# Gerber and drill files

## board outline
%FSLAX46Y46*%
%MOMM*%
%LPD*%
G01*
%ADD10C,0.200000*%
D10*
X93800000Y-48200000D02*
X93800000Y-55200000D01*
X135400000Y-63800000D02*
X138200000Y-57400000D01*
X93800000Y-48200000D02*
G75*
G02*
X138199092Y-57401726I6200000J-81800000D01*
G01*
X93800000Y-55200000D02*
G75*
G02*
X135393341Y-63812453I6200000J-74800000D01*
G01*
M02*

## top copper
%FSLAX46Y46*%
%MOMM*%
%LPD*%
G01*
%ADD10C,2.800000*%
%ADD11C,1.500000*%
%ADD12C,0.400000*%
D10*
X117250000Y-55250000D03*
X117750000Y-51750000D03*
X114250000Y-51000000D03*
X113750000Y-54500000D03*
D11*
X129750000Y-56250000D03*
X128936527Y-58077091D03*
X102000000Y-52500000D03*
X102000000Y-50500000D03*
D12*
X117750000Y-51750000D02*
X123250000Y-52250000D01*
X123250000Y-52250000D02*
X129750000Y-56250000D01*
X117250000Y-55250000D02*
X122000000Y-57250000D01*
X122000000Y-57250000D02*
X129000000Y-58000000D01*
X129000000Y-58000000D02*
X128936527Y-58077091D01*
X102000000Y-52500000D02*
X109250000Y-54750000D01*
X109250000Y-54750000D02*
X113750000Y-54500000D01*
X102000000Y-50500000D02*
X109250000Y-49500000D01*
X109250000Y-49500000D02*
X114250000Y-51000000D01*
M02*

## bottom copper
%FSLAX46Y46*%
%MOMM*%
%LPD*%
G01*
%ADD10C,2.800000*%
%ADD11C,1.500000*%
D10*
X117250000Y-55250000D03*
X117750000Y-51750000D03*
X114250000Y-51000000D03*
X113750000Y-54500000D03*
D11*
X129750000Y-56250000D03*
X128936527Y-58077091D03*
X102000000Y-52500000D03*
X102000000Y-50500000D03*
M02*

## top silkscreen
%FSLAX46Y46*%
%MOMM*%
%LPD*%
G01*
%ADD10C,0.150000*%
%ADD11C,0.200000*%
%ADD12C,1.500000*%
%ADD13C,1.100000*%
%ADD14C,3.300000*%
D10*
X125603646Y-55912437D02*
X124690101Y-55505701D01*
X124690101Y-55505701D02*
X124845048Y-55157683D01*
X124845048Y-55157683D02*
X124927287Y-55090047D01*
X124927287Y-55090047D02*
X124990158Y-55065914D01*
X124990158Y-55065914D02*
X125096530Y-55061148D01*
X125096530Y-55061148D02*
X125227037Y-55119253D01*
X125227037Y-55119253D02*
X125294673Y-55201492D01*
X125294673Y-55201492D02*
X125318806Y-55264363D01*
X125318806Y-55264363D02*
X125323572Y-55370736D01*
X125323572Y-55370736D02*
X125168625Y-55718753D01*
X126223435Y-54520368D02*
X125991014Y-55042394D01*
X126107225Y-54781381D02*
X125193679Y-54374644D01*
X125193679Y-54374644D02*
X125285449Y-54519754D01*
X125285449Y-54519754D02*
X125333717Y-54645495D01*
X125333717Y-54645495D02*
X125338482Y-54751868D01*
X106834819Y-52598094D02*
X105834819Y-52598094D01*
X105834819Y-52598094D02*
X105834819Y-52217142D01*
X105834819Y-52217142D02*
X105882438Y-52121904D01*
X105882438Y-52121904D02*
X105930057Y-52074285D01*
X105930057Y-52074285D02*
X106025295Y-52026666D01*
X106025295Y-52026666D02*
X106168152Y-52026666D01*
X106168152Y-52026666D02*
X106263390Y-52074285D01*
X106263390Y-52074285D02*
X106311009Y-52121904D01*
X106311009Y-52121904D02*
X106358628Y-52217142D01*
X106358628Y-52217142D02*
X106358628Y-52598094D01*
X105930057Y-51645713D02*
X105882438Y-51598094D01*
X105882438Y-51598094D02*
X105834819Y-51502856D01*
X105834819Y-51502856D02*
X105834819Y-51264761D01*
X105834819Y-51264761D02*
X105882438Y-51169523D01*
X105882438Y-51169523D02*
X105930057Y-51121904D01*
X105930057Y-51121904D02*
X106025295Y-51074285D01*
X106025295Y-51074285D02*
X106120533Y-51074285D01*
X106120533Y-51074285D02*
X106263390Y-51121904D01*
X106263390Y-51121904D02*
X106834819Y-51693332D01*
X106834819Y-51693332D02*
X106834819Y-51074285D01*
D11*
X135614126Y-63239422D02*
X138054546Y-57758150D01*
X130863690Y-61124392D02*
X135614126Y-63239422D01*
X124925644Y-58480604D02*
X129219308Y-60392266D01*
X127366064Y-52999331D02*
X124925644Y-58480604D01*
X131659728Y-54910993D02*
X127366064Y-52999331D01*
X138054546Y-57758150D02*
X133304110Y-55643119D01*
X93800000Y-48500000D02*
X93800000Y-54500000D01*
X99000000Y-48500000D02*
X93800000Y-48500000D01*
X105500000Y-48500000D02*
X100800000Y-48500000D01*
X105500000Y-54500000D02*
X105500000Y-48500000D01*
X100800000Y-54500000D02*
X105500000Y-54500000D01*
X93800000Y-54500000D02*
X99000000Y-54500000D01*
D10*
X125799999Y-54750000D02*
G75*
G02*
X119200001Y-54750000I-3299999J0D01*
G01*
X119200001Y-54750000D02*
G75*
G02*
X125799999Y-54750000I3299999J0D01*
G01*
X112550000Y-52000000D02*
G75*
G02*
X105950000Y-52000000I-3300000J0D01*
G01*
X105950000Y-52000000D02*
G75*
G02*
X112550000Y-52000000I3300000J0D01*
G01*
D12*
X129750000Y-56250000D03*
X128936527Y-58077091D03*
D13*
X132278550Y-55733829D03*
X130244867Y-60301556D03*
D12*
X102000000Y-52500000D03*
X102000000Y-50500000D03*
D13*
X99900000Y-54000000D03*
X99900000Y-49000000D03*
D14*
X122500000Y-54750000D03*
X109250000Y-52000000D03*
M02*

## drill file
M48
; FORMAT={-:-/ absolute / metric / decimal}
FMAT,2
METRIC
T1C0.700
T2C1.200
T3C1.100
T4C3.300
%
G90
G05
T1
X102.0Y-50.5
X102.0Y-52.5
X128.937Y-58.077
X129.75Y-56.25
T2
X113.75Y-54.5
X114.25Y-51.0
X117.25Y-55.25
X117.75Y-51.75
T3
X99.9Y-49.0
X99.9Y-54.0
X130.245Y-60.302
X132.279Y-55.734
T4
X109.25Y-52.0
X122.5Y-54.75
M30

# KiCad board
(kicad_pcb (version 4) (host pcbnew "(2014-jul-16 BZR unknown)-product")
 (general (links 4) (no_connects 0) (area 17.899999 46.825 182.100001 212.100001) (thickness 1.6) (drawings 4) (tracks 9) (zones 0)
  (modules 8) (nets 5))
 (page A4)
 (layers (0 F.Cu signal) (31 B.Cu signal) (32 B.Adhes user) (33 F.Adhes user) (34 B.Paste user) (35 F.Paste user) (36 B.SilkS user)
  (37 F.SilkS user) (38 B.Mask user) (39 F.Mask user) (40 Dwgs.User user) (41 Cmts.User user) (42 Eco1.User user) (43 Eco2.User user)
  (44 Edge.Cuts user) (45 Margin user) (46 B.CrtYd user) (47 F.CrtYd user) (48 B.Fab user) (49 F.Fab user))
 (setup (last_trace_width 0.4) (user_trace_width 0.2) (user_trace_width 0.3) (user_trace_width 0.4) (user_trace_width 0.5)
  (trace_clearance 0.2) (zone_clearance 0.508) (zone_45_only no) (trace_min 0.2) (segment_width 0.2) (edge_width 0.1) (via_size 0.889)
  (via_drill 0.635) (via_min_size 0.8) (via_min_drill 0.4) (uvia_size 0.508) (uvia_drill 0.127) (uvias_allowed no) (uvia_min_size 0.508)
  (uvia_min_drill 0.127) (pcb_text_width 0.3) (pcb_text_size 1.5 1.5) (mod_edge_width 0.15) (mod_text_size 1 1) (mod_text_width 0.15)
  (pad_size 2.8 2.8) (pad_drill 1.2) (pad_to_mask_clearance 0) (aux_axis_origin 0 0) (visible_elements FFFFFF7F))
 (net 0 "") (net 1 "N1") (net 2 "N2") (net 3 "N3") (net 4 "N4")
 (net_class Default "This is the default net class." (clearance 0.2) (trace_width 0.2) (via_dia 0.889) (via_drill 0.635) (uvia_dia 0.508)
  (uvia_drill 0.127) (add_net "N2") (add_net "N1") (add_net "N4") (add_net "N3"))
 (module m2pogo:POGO (layer F.Cu) (at 117.25 55.25)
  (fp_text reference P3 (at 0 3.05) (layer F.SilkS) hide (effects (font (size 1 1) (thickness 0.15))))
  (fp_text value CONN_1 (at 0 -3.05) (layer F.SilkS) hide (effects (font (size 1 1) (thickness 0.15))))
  (pad 1 thru_hole circle (at 0 0) (size 2.8 2.8) (drill 1.2) (layers *.Cu *.Mask) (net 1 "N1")))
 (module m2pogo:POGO (layer F.Cu) (at 117.75 51.75)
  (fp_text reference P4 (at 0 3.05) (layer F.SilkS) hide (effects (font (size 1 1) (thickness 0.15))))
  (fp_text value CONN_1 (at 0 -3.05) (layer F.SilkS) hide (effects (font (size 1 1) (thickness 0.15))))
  (pad 1 thru_hole circle (at 0 0) (size 2.8 2.8) (drill 1.2) (layers *.Cu *.Mask) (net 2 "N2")))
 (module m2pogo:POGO (layer F.Cu) (at 114.25 51)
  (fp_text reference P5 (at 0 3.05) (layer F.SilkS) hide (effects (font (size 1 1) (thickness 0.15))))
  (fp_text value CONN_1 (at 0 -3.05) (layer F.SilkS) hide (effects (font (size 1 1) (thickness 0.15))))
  (pad 1 thru_hole circle (at 0 0) (size 2.8 2.8) (drill 1.2) (layers *.Cu *.Mask) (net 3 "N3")))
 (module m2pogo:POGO (layer F.Cu) (at 113.75 54.5)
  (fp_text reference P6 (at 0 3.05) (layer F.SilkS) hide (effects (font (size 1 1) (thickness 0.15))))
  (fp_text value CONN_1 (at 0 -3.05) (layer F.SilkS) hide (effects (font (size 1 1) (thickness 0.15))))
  (pad 1 thru_hole circle (at 0 0) (size 2.8 2.8) (drill 1.2) (layers *.Cu *.Mask) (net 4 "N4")))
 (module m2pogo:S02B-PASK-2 (layer F.Cu) (at 129.75 56.25 246)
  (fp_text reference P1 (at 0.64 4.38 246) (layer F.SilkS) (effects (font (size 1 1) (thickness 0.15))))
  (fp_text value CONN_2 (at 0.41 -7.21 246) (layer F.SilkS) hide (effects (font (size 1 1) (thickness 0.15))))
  (fp_line (start 4 -8.2) (end -2 -8.2) (layer F.SilkS) (width 0.2))
  (fp_line (start 4 -3) (end 4 -8.2) (layer F.SilkS) (width 0.2))
  (fp_line (start 4 3.5) (end 4 -1.2) (layer F.SilkS) (width 0.2))
  (fp_line (start -2 3.5) (end 4 3.5) (layer F.SilkS) (width 0.2))
  (fp_line (start -2 -1.2) (end -2 3.5) (layer F.SilkS) (width 0.2))
  (fp_line (start -2 -8.2) (end -2 -3) (layer F.SilkS) (width 0.2))
  (pad 1 thru_hole circle (at 0 0 246) (size 1.5 1.5) (drill 0.7) (layers *.Cu *.Mask F.SilkS) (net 2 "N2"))
  (pad 2 thru_hole circle (at 2 0 246) (size 1.5 1.5) (drill 0.7) (layers *.Cu *.Mask F.SilkS) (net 1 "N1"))
  (pad "" np_thru_hole circle (at -1.5 -2.1 246) (size 1.1 1.1) (drill 1.1) (layers *.Cu *.Mask F.SilkS))
  (pad "" np_thru_hole circle (at 3.5 -2.1 246) (size 1.1 1.1) (drill 1.1) (layers *.Cu *.Mask F.SilkS)))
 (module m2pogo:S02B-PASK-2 (layer F.Cu) (at 102 52.5 90)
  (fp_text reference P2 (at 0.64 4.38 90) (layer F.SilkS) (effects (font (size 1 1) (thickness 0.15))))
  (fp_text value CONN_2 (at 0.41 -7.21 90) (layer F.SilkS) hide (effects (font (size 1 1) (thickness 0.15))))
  (fp_line (start 4 -8.2) (end -2 -8.2) (layer F.SilkS) (width 0.2))
  (fp_line (start 4 -3) (end 4 -8.2) (layer F.SilkS) (width 0.2))
  (fp_line (start 4 3.5) (end 4 -1.2) (layer F.SilkS) (width 0.2))
  (fp_line (start -2 3.5) (end 4 3.5) (layer F.SilkS) (width 0.2))
  (fp_line (start -2 -1.2) (end -2 3.5) (layer F.SilkS) (width 0.2))
  (fp_line (start -2 -8.2) (end -2 -3) (layer F.SilkS) (width 0.2))
  (pad 1 thru_hole circle (at 0 0 90) (size 1.5 1.5) (drill 0.7) (layers *.Cu *.Mask F.SilkS) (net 4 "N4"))
  (pad 2 thru_hole circle (at 2 0 90) (size 1.5 1.5) (drill 0.7) (layers *.Cu *.Mask F.SilkS) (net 3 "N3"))
  (pad "" np_thru_hole circle (at -1.5 -2.1 90) (size 1.1 1.1) (drill 1.1) (layers *.Cu *.Mask F.SilkS))
  (pad "" np_thru_hole circle (at 3.5 -2.1 90) (size 1.1 1.1) (drill 1.1) (layers *.Cu *.Mask F.SilkS)))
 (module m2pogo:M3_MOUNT (layer F.Cu) (at 122.5 54.75 67.5)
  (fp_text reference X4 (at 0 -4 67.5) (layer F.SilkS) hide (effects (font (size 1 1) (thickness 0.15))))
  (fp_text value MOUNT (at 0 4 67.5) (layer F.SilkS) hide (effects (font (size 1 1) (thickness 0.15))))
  (fp_circle (center 0 0) (end 3.3 0) (layer F.SilkS) (width 0.15))
  (pad "" np_thru_hole circle (at 0 0 67.5) (size 3.3 3.3) (drill 3.3) (layers *.Cu *.Mask F.Paste F.SilkS)))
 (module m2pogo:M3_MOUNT (layer F.Cu) (at 109.25 52)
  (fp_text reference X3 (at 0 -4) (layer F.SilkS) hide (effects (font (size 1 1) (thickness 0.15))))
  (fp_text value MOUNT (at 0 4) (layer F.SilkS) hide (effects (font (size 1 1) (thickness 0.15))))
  (fp_circle (center 0 0) (end 3.3 0) (layer F.SilkS) (width 0.15))
  (pad "" np_thru_hole circle (at 0 0) (size 3.3 3.3) (drill 3.3) (layers *.Cu *.Mask F.Paste F.SilkS)))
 (gr_line (start 93.8 48.2) (end 93.8 55.2) (layer Edge.Cuts) (width 0.2))
 (gr_line (start 135.4 63.8) (end 138.2 57.4) (layer Edge.Cuts) (width 0.2))
 (gr_arc (start 100 130) (end 93.8 48.2) (angle 32.08645929) (layer Edge.Cuts) (width 0.2))
 (gr_arc (start 100 130) (end 93.8 55.2) (angle 32.87362473) (layer Edge.Cuts) (width 0.2))
 (segment (start 117.75 51.75) (end 123.25 52.25) (width 0.4) (layer F.Cu) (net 2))
 (segment (start 123.25 52.25) (end 129.75 56.25) (width 0.4) (layer F.Cu) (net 2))
 (segment (start 117.25 55.25) (end 122 57.25) (width 0.4) (layer F.Cu) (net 1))
 (segment (start 122 57.25) (end 129 58) (width 0.4) (layer F.Cu) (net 1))
 (segment (start 129 58) (end 128.936527 58.077091) (width 0.4) (layer F.Cu) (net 1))
 (segment (start 102 52.5) (end 109.25 54.75) (width 0.4) (layer F.Cu) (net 4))
 (segment (start 109.25 54.75) (end 113.75 54.5) (width 0.4) (layer F.Cu) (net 4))
 (segment (start 102 50.5) (end 109.25 49.5) (width 0.4) (layer F.Cu) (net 3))
 (segment (start 109.25 49.5) (end 114.25 51) (width 0.4) (layer F.Cu) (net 3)))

